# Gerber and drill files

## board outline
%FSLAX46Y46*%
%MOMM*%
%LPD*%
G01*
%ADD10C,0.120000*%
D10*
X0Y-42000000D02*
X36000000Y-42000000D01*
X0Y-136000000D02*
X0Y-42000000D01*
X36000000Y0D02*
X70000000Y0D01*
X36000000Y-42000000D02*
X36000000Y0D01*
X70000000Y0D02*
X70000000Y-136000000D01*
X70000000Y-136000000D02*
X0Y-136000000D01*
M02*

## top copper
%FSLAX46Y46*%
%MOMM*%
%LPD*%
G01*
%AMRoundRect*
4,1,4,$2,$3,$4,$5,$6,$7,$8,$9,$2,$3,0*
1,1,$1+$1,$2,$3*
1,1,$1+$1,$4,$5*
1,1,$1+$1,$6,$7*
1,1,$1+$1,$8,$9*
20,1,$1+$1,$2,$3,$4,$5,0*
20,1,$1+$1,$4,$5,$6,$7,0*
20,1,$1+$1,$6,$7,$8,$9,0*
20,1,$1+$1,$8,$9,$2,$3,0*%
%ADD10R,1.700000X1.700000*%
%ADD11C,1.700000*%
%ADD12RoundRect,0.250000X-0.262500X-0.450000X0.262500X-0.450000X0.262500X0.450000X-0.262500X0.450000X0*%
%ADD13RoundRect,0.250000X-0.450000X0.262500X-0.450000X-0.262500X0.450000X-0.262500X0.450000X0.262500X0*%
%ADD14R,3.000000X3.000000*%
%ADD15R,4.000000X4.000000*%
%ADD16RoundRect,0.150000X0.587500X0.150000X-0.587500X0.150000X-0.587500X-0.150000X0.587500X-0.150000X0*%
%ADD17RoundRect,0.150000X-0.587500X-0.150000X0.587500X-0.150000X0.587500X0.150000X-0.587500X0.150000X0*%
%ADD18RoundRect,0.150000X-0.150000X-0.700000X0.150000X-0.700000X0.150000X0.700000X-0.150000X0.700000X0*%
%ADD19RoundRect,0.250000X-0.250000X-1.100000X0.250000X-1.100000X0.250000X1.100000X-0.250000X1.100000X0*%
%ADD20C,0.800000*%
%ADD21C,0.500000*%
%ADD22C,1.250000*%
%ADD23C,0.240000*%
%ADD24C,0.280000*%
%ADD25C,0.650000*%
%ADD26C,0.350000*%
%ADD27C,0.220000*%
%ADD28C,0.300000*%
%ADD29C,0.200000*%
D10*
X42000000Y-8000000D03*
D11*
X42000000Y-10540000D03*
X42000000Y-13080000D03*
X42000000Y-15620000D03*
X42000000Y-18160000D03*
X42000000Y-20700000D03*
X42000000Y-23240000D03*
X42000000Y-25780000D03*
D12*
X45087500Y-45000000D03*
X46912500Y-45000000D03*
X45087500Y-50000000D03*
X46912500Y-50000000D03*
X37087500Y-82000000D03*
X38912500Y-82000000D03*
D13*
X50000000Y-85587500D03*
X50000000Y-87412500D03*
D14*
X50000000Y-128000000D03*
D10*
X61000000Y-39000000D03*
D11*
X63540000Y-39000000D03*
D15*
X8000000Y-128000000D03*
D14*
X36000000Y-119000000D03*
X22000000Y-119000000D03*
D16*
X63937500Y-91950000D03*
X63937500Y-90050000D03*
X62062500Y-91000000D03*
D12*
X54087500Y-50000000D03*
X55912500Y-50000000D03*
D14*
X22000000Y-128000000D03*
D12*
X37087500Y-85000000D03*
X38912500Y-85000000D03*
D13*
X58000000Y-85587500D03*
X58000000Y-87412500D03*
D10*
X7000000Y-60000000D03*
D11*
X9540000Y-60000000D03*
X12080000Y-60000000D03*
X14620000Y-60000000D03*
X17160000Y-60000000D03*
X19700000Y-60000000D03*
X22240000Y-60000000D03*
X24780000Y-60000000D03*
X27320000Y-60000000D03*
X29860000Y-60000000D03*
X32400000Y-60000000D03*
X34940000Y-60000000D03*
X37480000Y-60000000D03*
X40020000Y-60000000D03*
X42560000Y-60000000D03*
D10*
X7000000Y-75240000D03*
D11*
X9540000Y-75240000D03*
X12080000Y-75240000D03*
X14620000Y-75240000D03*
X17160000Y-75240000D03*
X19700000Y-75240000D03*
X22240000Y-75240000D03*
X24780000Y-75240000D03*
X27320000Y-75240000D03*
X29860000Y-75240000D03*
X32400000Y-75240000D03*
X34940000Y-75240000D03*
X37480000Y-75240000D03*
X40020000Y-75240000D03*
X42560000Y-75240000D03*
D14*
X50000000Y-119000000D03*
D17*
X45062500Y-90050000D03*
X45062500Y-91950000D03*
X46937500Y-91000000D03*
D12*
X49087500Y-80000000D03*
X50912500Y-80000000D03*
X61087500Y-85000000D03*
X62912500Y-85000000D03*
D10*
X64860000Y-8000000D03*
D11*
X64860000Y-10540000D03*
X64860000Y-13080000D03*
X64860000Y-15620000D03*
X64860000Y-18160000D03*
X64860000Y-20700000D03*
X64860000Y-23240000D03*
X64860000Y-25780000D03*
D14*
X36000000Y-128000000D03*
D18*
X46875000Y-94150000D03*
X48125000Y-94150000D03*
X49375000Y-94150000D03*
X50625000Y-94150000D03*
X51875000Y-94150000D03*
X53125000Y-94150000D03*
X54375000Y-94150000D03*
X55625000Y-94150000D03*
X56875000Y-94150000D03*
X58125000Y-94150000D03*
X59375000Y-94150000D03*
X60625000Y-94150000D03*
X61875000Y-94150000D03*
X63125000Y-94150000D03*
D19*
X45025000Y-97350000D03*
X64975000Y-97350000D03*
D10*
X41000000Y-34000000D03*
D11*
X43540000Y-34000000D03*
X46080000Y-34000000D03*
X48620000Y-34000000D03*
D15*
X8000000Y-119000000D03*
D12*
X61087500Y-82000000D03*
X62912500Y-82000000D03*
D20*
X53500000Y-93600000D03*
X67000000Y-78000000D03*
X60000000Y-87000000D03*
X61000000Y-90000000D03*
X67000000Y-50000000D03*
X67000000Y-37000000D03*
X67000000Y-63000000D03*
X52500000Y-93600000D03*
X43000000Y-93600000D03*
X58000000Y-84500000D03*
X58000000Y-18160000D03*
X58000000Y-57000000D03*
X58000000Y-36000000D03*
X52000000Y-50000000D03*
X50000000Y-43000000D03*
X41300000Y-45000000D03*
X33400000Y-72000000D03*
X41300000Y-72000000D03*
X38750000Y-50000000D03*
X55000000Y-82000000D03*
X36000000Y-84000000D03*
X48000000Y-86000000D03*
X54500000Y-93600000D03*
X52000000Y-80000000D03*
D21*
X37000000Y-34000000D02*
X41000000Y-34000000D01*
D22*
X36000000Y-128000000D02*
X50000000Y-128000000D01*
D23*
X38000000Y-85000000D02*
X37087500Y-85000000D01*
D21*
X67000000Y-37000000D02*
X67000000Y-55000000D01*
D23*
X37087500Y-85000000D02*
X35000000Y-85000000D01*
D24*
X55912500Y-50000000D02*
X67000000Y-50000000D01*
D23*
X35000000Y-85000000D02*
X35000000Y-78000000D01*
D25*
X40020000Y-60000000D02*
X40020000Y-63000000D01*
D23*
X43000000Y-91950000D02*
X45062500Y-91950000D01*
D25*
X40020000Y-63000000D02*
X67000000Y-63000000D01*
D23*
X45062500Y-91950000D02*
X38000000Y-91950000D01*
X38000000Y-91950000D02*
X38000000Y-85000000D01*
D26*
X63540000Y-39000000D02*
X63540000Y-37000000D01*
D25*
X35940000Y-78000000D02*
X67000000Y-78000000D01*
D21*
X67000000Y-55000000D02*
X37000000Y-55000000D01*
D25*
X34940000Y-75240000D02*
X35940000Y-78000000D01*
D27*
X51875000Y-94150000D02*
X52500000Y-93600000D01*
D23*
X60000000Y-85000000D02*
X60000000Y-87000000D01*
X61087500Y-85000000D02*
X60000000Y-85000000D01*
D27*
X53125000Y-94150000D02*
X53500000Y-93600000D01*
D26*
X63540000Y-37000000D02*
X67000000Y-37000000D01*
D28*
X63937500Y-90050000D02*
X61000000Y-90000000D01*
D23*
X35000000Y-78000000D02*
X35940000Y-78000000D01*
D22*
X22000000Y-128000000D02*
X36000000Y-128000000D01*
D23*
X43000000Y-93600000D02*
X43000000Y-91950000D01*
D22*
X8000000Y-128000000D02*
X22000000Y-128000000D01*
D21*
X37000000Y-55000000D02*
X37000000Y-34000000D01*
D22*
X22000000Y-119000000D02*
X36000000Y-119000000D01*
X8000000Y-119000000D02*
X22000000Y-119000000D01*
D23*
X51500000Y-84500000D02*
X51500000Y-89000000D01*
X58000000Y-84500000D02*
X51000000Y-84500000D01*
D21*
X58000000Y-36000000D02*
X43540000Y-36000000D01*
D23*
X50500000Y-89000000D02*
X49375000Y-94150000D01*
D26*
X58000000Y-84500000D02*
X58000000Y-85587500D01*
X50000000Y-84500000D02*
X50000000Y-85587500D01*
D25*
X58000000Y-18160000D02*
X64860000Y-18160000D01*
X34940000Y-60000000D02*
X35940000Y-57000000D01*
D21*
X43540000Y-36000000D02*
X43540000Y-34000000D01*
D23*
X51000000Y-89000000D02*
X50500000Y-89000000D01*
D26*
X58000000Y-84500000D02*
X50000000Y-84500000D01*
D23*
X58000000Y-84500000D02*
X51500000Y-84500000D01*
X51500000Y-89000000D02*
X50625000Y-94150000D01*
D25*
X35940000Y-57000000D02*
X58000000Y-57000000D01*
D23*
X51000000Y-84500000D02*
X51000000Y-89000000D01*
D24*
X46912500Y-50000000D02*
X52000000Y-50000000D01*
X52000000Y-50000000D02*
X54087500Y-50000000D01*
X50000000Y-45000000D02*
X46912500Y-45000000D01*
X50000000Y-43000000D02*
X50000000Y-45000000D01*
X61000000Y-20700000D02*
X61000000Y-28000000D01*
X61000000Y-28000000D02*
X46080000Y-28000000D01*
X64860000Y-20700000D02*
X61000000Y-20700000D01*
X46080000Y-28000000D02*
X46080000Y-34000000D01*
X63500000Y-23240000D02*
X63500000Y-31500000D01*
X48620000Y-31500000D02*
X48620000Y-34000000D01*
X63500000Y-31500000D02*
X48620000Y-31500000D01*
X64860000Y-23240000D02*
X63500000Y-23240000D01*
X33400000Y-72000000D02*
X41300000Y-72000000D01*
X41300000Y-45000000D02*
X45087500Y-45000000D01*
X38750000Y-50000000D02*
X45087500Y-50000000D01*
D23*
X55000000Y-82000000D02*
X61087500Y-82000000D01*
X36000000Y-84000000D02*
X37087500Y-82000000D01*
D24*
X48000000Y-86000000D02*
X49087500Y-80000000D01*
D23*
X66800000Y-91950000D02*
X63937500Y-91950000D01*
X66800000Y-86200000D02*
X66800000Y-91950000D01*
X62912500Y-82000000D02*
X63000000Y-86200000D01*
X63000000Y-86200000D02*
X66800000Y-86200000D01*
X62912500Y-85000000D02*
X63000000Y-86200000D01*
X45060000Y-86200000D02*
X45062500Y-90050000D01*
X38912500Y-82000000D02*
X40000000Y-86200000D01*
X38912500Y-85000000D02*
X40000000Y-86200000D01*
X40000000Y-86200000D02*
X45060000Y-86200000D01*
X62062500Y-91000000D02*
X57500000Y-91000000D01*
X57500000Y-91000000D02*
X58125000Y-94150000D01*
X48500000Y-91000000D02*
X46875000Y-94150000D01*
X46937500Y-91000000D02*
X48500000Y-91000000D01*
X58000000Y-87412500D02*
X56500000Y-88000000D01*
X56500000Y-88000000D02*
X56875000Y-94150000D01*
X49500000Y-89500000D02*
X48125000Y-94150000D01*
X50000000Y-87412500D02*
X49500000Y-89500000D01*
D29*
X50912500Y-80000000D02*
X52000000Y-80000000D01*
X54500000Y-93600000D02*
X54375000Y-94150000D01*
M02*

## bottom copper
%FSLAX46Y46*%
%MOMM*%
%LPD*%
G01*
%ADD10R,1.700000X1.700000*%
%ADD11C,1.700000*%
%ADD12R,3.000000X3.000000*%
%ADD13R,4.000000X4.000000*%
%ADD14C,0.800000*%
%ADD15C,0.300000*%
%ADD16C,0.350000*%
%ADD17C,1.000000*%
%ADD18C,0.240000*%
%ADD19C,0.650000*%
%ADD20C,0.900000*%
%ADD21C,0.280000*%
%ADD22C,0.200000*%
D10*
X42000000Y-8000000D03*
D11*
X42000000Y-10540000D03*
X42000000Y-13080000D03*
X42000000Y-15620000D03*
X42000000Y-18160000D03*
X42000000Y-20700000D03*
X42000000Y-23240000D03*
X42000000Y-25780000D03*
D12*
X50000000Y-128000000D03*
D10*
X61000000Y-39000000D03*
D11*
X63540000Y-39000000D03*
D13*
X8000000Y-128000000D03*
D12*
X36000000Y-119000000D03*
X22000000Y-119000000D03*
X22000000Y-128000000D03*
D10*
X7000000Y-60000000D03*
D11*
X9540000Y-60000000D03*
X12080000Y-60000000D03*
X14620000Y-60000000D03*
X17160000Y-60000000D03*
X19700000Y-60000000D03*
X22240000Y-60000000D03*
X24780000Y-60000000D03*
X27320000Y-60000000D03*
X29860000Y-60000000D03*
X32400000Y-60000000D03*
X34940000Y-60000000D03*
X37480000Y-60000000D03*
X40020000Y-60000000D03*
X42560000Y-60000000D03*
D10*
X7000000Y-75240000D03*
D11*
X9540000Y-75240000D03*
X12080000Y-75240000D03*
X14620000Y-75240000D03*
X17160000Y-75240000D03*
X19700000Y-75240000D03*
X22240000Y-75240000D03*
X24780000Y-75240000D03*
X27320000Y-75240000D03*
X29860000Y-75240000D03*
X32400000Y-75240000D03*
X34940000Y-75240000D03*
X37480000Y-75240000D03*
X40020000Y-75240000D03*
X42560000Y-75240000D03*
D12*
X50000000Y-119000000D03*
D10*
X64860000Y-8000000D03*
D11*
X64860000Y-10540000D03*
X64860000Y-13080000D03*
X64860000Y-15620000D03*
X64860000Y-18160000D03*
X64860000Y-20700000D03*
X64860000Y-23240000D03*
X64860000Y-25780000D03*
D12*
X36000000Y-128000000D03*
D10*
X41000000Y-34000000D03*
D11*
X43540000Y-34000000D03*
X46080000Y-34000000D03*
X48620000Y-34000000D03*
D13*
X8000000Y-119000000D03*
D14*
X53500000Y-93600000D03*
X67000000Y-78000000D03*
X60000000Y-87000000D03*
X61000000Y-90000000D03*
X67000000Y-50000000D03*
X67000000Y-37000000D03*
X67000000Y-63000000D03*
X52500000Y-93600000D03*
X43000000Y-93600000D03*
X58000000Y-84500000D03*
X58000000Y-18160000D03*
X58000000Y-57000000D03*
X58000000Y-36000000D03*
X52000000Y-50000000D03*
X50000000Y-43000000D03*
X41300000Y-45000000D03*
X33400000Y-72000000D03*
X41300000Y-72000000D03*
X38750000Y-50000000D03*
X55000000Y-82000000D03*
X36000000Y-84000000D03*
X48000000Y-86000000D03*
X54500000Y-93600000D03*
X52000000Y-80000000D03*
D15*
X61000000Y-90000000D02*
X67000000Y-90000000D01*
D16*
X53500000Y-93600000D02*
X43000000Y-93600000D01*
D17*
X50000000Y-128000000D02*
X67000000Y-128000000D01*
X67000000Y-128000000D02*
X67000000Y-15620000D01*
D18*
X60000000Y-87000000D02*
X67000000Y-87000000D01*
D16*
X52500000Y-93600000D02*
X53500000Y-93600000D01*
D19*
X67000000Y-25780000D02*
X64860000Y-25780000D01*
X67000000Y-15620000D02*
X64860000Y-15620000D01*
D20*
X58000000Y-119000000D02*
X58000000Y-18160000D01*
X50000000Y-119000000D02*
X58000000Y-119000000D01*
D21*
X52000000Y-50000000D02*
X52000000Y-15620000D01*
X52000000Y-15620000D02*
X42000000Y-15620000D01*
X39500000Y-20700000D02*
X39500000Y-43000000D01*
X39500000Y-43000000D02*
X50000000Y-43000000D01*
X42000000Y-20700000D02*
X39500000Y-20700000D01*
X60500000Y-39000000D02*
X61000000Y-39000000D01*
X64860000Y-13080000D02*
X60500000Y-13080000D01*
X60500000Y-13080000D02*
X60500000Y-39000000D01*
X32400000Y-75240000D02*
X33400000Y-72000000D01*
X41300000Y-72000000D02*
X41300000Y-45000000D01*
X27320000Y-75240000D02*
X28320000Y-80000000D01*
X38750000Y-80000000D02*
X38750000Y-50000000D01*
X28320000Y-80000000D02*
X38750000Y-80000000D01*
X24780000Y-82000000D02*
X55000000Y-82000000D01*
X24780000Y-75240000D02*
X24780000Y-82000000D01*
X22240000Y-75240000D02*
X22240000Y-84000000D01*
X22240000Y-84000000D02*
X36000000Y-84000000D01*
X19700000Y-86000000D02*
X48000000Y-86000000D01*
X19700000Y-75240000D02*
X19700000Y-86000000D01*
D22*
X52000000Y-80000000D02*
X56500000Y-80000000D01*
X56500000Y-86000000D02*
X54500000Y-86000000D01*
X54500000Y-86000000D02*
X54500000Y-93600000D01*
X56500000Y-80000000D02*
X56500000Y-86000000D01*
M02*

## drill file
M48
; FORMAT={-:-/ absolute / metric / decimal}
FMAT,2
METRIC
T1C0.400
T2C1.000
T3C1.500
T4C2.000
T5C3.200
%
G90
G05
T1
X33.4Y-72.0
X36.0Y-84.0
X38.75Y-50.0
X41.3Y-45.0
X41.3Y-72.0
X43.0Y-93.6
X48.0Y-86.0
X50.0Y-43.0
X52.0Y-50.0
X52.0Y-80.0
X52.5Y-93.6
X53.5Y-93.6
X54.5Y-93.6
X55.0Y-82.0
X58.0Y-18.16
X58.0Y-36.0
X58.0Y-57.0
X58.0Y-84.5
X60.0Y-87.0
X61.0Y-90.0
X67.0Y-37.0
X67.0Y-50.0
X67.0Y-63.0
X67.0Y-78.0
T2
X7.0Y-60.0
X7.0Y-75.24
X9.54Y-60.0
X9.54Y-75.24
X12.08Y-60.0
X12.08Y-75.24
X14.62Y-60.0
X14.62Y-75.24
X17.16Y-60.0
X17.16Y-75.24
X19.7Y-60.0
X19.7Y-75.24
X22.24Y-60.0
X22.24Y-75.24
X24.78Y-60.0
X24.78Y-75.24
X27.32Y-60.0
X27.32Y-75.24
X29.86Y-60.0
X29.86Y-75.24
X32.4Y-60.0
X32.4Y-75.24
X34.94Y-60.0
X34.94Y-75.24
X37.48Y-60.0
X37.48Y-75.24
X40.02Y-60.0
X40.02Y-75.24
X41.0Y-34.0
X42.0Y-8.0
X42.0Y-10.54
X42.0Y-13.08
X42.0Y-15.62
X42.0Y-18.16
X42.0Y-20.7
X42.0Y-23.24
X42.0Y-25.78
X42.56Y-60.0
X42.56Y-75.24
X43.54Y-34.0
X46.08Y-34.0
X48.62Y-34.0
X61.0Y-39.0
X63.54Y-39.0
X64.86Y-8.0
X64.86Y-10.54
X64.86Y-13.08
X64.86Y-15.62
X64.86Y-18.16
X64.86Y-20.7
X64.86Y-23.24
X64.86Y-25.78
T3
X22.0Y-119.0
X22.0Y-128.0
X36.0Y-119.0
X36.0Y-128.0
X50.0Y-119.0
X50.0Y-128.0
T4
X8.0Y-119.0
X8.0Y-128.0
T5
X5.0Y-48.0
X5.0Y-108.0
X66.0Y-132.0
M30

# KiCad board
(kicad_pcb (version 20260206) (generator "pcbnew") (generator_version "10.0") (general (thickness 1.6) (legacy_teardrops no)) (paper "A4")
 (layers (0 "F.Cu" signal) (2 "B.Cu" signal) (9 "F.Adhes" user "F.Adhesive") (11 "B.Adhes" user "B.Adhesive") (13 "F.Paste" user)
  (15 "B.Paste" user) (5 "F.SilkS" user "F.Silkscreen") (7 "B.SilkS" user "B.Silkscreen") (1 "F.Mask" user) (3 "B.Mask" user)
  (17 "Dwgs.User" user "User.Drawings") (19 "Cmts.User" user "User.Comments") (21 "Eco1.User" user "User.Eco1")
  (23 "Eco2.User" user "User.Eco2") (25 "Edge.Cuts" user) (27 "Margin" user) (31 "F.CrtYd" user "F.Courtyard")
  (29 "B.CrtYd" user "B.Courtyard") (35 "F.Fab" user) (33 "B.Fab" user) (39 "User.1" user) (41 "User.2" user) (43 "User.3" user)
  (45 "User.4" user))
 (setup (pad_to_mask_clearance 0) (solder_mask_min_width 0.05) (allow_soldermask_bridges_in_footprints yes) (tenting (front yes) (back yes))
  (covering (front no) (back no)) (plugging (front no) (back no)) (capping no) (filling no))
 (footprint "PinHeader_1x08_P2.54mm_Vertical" (layer "F.Cu") (at 42 8)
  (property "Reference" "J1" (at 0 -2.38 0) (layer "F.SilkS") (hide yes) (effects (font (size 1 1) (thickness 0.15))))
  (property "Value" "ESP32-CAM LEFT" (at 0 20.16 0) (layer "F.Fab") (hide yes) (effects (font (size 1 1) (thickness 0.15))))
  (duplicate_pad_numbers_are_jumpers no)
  (pad "1" thru_hole rect (at 0 0) (size 1.7 1.7) (drill 1) (layers "*.Cu" "*.Mask") (remove_unused_layers no))
  (pad "2" thru_hole circle (at 0 2.54) (size 1.7 1.7) (drill 1) (layers "*.Cu" "*.Mask") (remove_unused_layers no))
  (pad "3" thru_hole circle (at 0 5.08) (size 1.7 1.7) (drill 1) (layers "*.Cu" "*.Mask") (remove_unused_layers no))
  (pad "4" thru_hole circle (at 0 7.62) (size 1.7 1.7) (drill 1) (layers "*.Cu" "*.Mask") (remove_unused_layers no) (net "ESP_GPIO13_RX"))
  (pad "5" thru_hole circle (at 0 10.16) (size 1.7 1.7) (drill 1) (layers "*.Cu" "*.Mask") (remove_unused_layers no))
  (pad "6" thru_hole circle (at 0 12.7) (size 1.7 1.7) (drill 1) (layers "*.Cu" "*.Mask") (remove_unused_layers no) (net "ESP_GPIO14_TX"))
  (pad "7" thru_hole circle (at 0 15.24) (size 1.7 1.7) (drill 1) (layers "*.Cu" "*.Mask") (remove_unused_layers no))
  (pad "8" thru_hole circle (at 0 17.78) (size 1.7 1.7) (drill 1) (layers "*.Cu" "*.Mask") (remove_unused_layers no)))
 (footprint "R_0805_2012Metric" (layer "F.Cu") (at 46 45)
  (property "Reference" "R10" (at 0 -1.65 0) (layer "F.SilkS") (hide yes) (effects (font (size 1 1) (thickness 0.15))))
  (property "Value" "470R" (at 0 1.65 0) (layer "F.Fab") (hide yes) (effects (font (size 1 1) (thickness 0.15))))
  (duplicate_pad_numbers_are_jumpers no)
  (pad "1" smd roundrect (at -0.9125 0) (size 1.025 1.4) (layers "F.Cu" "F.Mask" "F.Paste") (roundrect_rratio 0.243902) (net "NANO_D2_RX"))
  (pad "2" smd roundrect (at 0.9125 0) (size 1.025 1.4) (layers "F.Cu" "F.Mask" "F.Paste") (roundrect_rratio 0.243902) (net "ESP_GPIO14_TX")))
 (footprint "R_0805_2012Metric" (layer "F.Cu") (at 46 50)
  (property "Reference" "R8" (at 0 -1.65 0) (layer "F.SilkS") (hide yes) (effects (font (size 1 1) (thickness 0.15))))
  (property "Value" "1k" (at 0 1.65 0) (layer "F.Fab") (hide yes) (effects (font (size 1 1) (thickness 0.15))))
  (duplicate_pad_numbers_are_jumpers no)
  (pad "1" smd roundrect (at -0.9125 0) (size 1.025 1.4) (layers "F.Cu" "F.Mask" "F.Paste") (roundrect_rratio 0.243902) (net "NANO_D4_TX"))
  (pad "2" smd roundrect (at 0.9125 0) (size 1.025 1.4) (layers "F.Cu" "F.Mask" "F.Paste") (roundrect_rratio 0.243902) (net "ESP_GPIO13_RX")))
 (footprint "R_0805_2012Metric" (layer "F.Cu") (at 38 82)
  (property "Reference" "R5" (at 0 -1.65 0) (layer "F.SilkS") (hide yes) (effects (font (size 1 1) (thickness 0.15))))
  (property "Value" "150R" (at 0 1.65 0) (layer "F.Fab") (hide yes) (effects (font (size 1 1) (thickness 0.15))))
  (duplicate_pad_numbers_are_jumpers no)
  (pad "1" smd roundrect (at -0.9125 0) (size 1.025 1.4) (layers "F.Cu" "F.Mask" "F.Paste") (roundrect_rratio 0.243902)
   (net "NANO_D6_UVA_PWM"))
  (pad "2" smd roundrect (at 0.9125 0) (size 1.025 1.4) (layers "F.Cu" "F.Mask" "F.Paste") (roundrect_rratio 0.243902) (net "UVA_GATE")))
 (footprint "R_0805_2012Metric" (layer "F.Cu") (at 50 86.5 -90)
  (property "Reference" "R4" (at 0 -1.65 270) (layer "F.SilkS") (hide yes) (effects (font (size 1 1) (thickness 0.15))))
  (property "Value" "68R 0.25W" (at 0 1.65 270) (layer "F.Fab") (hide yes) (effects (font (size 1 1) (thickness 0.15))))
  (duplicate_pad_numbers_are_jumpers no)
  (pad "1" smd roundrect (at -0.9125 0 270) (size 1.025 1.4) (layers "F.Cu" "F.Mask" "F.Paste") (roundrect_rratio 0.243902) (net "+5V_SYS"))
  (pad "2" smd roundrect (at 0.9125 0 270) (size 1.025 1.4) (layers "F.Cu" "F.Mask" "F.Paste") (roundrect_rratio 0.243902) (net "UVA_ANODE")))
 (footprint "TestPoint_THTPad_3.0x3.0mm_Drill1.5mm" (layer "F.Cu") (at 50 128)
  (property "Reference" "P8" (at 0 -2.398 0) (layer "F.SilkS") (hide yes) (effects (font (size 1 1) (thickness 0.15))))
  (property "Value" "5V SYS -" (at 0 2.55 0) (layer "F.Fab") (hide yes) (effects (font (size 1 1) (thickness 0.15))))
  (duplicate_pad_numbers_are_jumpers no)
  (pad "1" thru_hole rect (at 0 0) (size 3 3) (drill 1.5) (layers "*.Cu" "*.Mask") (remove_unused_layers no) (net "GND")))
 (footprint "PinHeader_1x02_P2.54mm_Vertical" (layer "F.Cu") (at 61 39 90)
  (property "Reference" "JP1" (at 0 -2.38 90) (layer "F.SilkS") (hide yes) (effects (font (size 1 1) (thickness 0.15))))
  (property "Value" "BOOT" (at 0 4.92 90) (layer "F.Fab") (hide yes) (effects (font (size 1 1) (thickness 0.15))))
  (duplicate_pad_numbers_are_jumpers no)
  (pad "1" thru_hole rect (at 0 0 90) (size 1.7 1.7) (drill 1) (layers "*.Cu" "*.Mask") (remove_unused_layers no) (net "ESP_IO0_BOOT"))
  (pad "2" thru_hole circle (at 0 2.54 90) (size 1.7 1.7) (drill 1) (layers "*.Cu" "*.Mask") (remove_unused_layers no) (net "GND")))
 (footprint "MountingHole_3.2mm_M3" (layer "F.Cu") (at 5 108)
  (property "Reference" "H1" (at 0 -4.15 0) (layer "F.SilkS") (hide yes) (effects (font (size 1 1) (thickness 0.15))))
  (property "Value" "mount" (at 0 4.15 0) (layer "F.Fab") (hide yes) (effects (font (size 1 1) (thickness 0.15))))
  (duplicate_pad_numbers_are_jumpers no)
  (pad "" np_thru_hole circle (at 0 0) (size 3.2 3.2) (drill 3.2) (layers "*.Cu" "*.Mask")))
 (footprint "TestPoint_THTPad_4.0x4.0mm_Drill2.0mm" (layer "F.Cu") (at 8 128)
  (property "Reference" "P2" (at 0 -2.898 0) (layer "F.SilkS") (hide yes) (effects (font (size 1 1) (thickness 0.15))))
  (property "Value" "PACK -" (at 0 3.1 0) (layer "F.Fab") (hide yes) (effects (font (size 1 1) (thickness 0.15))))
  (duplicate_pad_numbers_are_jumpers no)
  (pad "1" thru_hole rect (at 0 0) (size 4 4) (drill 2) (layers "*.Cu" "*.Mask") (remove_unused_layers no) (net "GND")))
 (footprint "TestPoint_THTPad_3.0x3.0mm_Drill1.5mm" (layer "F.Cu") (at 36 119)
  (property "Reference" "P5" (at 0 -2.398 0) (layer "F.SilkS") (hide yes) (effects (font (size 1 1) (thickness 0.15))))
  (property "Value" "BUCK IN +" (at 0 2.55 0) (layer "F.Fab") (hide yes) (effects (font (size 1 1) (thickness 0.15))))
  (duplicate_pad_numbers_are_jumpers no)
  (pad "1" thru_hole rect (at 0 0) (size 3 3) (drill 1.5) (layers "*.Cu" "*.Mask") (remove_unused_layers no) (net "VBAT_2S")))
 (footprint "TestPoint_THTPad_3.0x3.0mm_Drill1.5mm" (layer "F.Cu") (at 22 119)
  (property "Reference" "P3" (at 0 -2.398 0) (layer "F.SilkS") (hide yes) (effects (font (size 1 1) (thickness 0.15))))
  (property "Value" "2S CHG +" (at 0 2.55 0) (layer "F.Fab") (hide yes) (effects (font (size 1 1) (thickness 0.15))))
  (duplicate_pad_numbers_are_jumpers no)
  (pad "1" thru_hole rect (at 0 0) (size 3 3) (drill 1.5) (layers "*.Cu" "*.Mask") (remove_unused_layers no) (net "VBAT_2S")))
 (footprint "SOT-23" (layer "F.Cu") (at 63 91 180)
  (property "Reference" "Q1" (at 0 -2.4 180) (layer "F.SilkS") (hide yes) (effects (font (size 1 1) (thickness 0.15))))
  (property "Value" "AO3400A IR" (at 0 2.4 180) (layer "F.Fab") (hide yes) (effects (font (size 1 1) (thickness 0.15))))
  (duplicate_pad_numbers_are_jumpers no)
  (pad "1" smd roundrect (at -0.9375 -0.95 180) (size 1.475 0.6) (layers "F.Cu" "F.Mask" "F.Paste") (roundrect_rratio 0.25) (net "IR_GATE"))
  (pad "2" smd roundrect (at -0.9375 0.95 180) (size 1.475 0.6) (layers "F.Cu" "F.Mask" "F.Paste") (roundrect_rratio 0.25) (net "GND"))
  (pad "3" smd roundrect (at 0.9375 0 180) (size 1.475 0.6) (layers "F.Cu" "F.Mask" "F.Paste") (roundrect_rratio 0.25) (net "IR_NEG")))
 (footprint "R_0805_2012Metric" (layer "F.Cu") (at 55 50)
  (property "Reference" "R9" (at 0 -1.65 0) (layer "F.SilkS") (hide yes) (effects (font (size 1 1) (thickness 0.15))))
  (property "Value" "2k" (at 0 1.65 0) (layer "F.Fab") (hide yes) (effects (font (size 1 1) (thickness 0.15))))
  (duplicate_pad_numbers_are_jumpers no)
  (pad "1" smd roundrect (at -0.9125 0) (size 1.025 1.4) (layers "F.Cu" "F.Mask" "F.Paste") (roundrect_rratio 0.243902)
   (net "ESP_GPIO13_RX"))
  (pad "2" smd roundrect (at 0.9125 0) (size 1.025 1.4) (layers "F.Cu" "F.Mask" "F.Paste") (roundrect_rratio 0.243902) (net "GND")))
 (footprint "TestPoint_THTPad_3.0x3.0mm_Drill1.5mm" (layer "F.Cu") (at 22 128)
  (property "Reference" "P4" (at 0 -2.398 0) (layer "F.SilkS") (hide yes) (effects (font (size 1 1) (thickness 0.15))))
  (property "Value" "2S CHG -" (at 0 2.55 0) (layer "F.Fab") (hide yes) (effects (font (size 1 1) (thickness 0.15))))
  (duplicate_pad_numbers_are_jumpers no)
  (pad "1" thru_hole rect (at 0 0) (size 3 3) (drill 1.5) (layers "*.Cu" "*.Mask") (remove_unused_layers no) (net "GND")))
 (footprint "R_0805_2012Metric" (layer "F.Cu") (at 38 85)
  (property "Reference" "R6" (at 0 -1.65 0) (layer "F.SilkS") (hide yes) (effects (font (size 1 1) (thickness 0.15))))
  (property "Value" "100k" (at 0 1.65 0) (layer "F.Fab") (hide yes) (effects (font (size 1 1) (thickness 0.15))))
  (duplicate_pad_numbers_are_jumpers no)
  (pad "1" smd roundrect (at -0.9125 0) (size 1.025 1.4) (layers "F.Cu" "F.Mask" "F.Paste") (roundrect_rratio 0.243902) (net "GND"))
  (pad "2" smd roundrect (at 0.9125 0) (size 1.025 1.4) (layers "F.Cu" "F.Mask" "F.Paste") (roundrect_rratio 0.243902) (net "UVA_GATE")))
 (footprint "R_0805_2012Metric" (layer "F.Cu") (at 58 86.5 -90)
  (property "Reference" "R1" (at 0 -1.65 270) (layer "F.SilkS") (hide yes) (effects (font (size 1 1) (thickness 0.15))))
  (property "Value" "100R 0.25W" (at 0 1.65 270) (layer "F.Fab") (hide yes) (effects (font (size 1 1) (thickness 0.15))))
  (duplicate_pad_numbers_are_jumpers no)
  (pad "1" smd roundrect (at -0.9125 0 270) (size 1.025 1.4) (layers "F.Cu" "F.Mask" "F.Paste") (roundrect_rratio 0.243902) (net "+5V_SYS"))
  (pad "2" smd roundrect (at 0.9125 0 270) (size 1.025 1.4) (layers "F.Cu" "F.Mask" "F.Paste") (roundrect_rratio 0.243902) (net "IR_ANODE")))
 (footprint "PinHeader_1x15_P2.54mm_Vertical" (layer "F.Cu") (at 7 60 90)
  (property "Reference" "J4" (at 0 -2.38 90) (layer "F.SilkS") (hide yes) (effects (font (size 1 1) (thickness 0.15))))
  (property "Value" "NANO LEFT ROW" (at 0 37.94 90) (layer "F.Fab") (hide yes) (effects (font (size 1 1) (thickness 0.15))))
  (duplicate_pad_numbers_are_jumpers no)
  (pad "1" thru_hole rect (at 0 0 90) (size 1.7 1.7) (drill 1) (layers "*.Cu" "*.Mask") (remove_unused_layers no))
  (pad "2" thru_hole circle (at 0 2.54 90) (size 1.7 1.7) (drill 1) (layers "*.Cu" "*.Mask") (remove_unused_layers no))
  (pad "3" thru_hole circle (at 0 5.08 90) (size 1.7 1.7) (drill 1) (layers "*.Cu" "*.Mask") (remove_unused_layers no))
  (pad "4" thru_hole circle (at 0 7.62 90) (size 1.7 1.7) (drill 1) (layers "*.Cu" "*.Mask") (remove_unused_layers no))
  (pad "5" thru_hole circle (at 0 10.16 90) (size 1.7 1.7) (drill 1) (layers "*.Cu" "*.Mask") (remove_unused_layers no))
  (pad "6" thru_hole circle (at 0 12.7 90) (size 1.7 1.7) (drill 1) (layers "*.Cu" "*.Mask") (remove_unused_layers no))
  (pad "7" thru_hole circle (at 0 15.24 90) (size 1.7 1.7) (drill 1) (layers "*.Cu" "*.Mask") (remove_unused_layers no))
  (pad "8" thru_hole circle (at 0 17.78 90) (size 1.7 1.7) (drill 1) (layers "*.Cu" "*.Mask") (remove_unused_layers no))
  (pad "9" thru_hole circle (at 0 20.32 90) (size 1.7 1.7) (drill 1) (layers "*.Cu" "*.Mask") (remove_unused_layers no))
  (pad "10" thru_hole circle (at 0 22.86 90) (size 1.7 1.7) (drill 1) (layers "*.Cu" "*.Mask") (remove_unused_layers no))
  (pad "11" thru_hole circle (at 0 25.4 90) (size 1.7 1.7) (drill 1) (layers "*.Cu" "*.Mask") (remove_unused_layers no))
  (pad "12" thru_hole circle (at 0 27.94 90) (size 1.7 1.7) (drill 1) (layers "*.Cu" "*.Mask") (remove_unused_layers no) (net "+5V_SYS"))
  (pad "13" thru_hole circle (at 0 30.48 90) (size 1.7 1.7) (drill 1) (layers "*.Cu" "*.Mask") (remove_unused_layers no))
  (pad "14" thru_hole circle (at 0 33.02 90) (size 1.7 1.7) (drill 1) (layers "*.Cu" "*.Mask") (remove_unused_layers no) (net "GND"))
  (pad "15" thru_hole circle (at 0 35.56 90) (size 1.7 1.7) (drill 1) (layers "*.Cu" "*.Mask") (remove_unused_layers no)))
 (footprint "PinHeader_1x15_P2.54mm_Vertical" (layer "F.Cu") (at 7 75.24 90)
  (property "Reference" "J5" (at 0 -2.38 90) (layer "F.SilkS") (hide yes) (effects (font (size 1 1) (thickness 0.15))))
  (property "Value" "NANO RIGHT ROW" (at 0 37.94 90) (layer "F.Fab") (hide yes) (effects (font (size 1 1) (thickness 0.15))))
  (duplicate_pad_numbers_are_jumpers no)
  (pad "1" thru_hole rect (at 0 0 90) (size 1.7 1.7) (drill 1) (layers "*.Cu" "*.Mask") (remove_unused_layers no))
  (pad "2" thru_hole circle (at 0 2.54 90) (size 1.7 1.7) (drill 1) (layers "*.Cu" "*.Mask") (remove_unused_layers no))
  (pad "3" thru_hole circle (at 0 5.08 90) (size 1.7 1.7) (drill 1) (layers "*.Cu" "*.Mask") (remove_unused_layers no))
  (pad "4" thru_hole circle (at 0 7.62 90) (size 1.7 1.7) (drill 1) (layers "*.Cu" "*.Mask") (remove_unused_layers no))
  (pad "5" thru_hole circle (at 0 10.16 90) (size 1.7 1.7) (drill 1) (layers "*.Cu" "*.Mask") (remove_unused_layers no)
   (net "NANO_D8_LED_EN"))
  (pad "6" thru_hole circle (at 0 12.7 90) (size 1.7 1.7) (drill 1) (layers "*.Cu" "*.Mask") (remove_unused_layers no)
   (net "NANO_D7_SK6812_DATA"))
  (pad "7" thru_hole circle (at 0 15.24 90) (size 1.7 1.7) (drill 1) (layers "*.Cu" "*.Mask") (remove_unused_layers no)
   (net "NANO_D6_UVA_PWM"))
  (pad "8" thru_hole circle (at 0 17.78 90) (size 1.7 1.7) (drill 1) (layers "*.Cu" "*.Mask") (remove_unused_layers no)
   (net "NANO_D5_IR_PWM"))
  (pad "9" thru_hole circle (at 0 20.32 90) (size 1.7 1.7) (drill 1) (layers "*.Cu" "*.Mask") (remove_unused_layers no) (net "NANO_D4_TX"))
  (pad "10" thru_hole circle (at 0 22.86 90) (size 1.7 1.7) (drill 1) (layers "*.Cu" "*.Mask") (remove_unused_layers no))
  (pad "11" thru_hole circle (at 0 25.4 90) (size 1.7 1.7) (drill 1) (layers "*.Cu" "*.Mask") (remove_unused_layers no) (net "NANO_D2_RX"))
  (pad "12" thru_hole circle (at 0 27.94 90) (size 1.7 1.7) (drill 1) (layers "*.Cu" "*.Mask") (remove_unused_layers no) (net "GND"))
  (pad "13" thru_hole circle (at 0 30.48 90) (size 1.7 1.7) (drill 1) (layers "*.Cu" "*.Mask") (remove_unused_layers no))
  (pad "14" thru_hole circle (at 0 33.02 90) (size 1.7 1.7) (drill 1) (layers "*.Cu" "*.Mask") (remove_unused_layers no))
  (pad "15" thru_hole circle (at 0 35.56 90) (size 1.7 1.7) (drill 1) (layers "*.Cu" "*.Mask") (remove_unused_layers no)))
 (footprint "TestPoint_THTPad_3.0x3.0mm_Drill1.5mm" (layer "F.Cu") (at 50 119)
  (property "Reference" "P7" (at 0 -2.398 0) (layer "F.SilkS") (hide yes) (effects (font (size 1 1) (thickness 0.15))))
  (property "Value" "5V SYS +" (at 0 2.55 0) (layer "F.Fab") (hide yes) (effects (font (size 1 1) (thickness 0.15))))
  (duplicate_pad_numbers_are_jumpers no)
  (pad "1" thru_hole rect (at 0 0) (size 3 3) (drill 1.5) (layers "*.Cu" "*.Mask") (remove_unused_layers no) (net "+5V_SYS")))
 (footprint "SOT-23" (layer "F.Cu") (at 46 91)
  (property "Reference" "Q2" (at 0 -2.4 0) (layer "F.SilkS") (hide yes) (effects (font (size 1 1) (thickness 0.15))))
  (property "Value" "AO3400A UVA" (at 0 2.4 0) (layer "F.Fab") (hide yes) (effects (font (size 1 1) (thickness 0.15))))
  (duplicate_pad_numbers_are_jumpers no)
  (pad "1" smd roundrect (at -0.9375 -0.95) (size 1.475 0.6) (layers "F.Cu" "F.Mask" "F.Paste") (roundrect_rratio 0.25) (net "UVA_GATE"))
  (pad "2" smd roundrect (at -0.9375 0.95) (size 1.475 0.6) (layers "F.Cu" "F.Mask" "F.Paste") (roundrect_rratio 0.25) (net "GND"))
  (pad "3" smd roundrect (at 0.9375 0) (size 1.475 0.6) (layers "F.Cu" "F.Mask" "F.Paste") (roundrect_rratio 0.25) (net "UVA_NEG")))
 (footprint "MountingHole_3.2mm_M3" (layer "F.Cu") (at 66 132)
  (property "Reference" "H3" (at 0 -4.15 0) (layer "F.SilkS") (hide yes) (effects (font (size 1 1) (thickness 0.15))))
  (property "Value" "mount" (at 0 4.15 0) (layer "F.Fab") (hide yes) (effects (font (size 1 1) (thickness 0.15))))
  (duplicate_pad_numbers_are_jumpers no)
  (pad "" np_thru_hole circle (at 0 0) (size 3.2 3.2) (drill 3.2) (layers "*.Cu" "*.Mask")))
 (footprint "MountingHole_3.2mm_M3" (layer "F.Cu") (at 5 48)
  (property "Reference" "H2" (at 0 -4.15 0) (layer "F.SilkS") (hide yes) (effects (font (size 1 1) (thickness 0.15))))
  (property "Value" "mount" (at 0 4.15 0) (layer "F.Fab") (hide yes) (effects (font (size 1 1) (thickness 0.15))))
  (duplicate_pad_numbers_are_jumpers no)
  (pad "" np_thru_hole circle (at 0 0) (size 3.2 3.2) (drill 3.2) (layers "*.Cu" "*.Mask")))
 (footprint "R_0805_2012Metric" (layer "F.Cu") (at 50 80)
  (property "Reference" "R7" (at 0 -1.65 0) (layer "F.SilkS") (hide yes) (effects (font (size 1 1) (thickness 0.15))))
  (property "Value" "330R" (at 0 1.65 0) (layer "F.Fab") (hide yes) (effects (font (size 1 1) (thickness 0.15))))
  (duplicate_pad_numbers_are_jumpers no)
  (pad "1" smd roundrect (at -0.9125 0) (size 1.025 1.4) (layers "F.Cu" "F.Mask" "F.Paste") (roundrect_rratio 0.243902)
   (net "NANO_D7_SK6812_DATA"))
  (pad "2" smd roundrect (at 0.9125 0) (size 1.025 1.4) (layers "F.Cu" "F.Mask" "F.Paste") (roundrect_rratio 0.243902) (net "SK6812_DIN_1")))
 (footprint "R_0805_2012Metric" (layer "F.Cu") (at 62 85)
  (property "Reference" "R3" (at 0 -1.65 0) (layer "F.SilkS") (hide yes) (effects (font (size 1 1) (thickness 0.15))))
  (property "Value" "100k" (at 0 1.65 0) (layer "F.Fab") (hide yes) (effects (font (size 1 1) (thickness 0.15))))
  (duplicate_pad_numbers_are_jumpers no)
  (pad "1" smd roundrect (at -0.9125 0) (size 1.025 1.4) (layers "F.Cu" "F.Mask" "F.Paste") (roundrect_rratio 0.243902) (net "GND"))
  (pad "2" smd roundrect (at 0.9125 0) (size 1.025 1.4) (layers "F.Cu" "F.Mask" "F.Paste") (roundrect_rratio 0.243902) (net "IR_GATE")))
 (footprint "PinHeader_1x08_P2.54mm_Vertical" (layer "F.Cu") (at 64.86 8)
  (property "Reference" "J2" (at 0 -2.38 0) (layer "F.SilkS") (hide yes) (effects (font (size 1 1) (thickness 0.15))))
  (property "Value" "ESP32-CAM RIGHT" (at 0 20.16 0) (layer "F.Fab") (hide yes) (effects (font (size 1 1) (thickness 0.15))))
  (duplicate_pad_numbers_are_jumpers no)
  (pad "1" thru_hole rect (at 0 0) (size 1.7 1.7) (drill 1) (layers "*.Cu" "*.Mask") (remove_unused_layers no))
  (pad "2" thru_hole circle (at 0 2.54) (size 1.7 1.7) (drill 1) (layers "*.Cu" "*.Mask") (remove_unused_layers no))
  (pad "3" thru_hole circle (at 0 5.08) (size 1.7 1.7) (drill 1) (layers "*.Cu" "*.Mask") (remove_unused_layers no) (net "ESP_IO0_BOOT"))
  (pad "4" thru_hole circle (at 0 7.62) (size 1.7 1.7) (drill 1) (layers "*.Cu" "*.Mask") (remove_unused_layers no) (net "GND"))
  (pad "5" thru_hole circle (at 0 10.16) (size 1.7 1.7) (drill 1) (layers "*.Cu" "*.Mask") (remove_unused_layers no) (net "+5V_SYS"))
  (pad "6" thru_hole circle (at 0 12.7) (size 1.7 1.7) (drill 1) (layers "*.Cu" "*.Mask") (remove_unused_layers no) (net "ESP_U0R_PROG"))
  (pad "7" thru_hole circle (at 0 15.24) (size 1.7 1.7) (drill 1) (layers "*.Cu" "*.Mask") (remove_unused_layers no) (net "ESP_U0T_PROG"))
  (pad "8" thru_hole circle (at 0 17.78) (size 1.7 1.7) (drill 1) (layers "*.Cu" "*.Mask") (remove_unused_layers no) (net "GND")))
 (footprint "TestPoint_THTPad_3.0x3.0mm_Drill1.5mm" (layer "F.Cu") (at 36 128)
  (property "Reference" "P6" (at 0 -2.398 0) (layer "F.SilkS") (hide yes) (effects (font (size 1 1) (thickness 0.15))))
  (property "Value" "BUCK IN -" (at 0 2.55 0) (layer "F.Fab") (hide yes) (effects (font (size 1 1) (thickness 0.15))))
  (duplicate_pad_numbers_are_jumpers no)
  (pad "1" thru_hole rect (at 0 0) (size 3 3) (drill 1.5) (layers "*.Cu" "*.Mask") (remove_unused_layers no) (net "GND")))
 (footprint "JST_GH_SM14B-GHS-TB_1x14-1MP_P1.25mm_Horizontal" (layer "F.Cu") (at 55 96)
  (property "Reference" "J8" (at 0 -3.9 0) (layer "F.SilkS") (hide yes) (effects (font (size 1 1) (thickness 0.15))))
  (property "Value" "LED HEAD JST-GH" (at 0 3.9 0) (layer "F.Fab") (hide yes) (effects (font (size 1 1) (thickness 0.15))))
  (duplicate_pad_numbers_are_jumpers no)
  (pad "1" smd roundrect (at -8.125 -1.85) (size 0.6 1.7) (layers "F.Cu" "F.Mask" "F.Paste") (roundrect_rratio 0.25) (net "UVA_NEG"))
  (pad "2" smd roundrect (at -6.875 -1.85) (size 0.6 1.7) (layers "F.Cu" "F.Mask" "F.Paste") (roundrect_rratio 0.25) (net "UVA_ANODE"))
  (pad "3" smd roundrect (at -5.625 -1.85) (size 0.6 1.7) (layers "F.Cu" "F.Mask" "F.Paste") (roundrect_rratio 0.25) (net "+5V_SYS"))
  (pad "4" smd roundrect (at -4.375 -1.85) (size 0.6 1.7) (layers "F.Cu" "F.Mask" "F.Paste") (roundrect_rratio 0.25) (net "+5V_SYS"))
  (pad "5" smd roundrect (at -3.125 -1.85) (size 0.6 1.7) (layers "F.Cu" "F.Mask" "F.Paste") (roundrect_rratio 0.25) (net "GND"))
  (pad "6" smd roundrect (at -1.875 -1.85) (size 0.6 1.7) (layers "F.Cu" "F.Mask" "F.Paste") (roundrect_rratio 0.25) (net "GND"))
  (pad "7" smd roundrect (at -0.625 -1.85) (size 0.6 1.7) (layers "F.Cu" "F.Mask" "F.Paste") (roundrect_rratio 0.25) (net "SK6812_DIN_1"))
  (pad "8" smd roundrect (at 0.625 -1.85) (size 0.6 1.7) (layers "F.Cu" "F.Mask" "F.Paste") (roundrect_rratio 0.25))
  (pad "9" smd roundrect (at 1.875 -1.85) (size 0.6 1.7) (layers "F.Cu" "F.Mask" "F.Paste") (roundrect_rratio 0.25) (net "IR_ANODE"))
  (pad "10" smd roundrect (at 3.125 -1.85) (size 0.6 1.7) (layers "F.Cu" "F.Mask" "F.Paste") (roundrect_rratio 0.25) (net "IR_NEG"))
  (pad "11" smd roundrect (at 4.375 -1.85) (size 0.6 1.7) (layers "F.Cu" "F.Mask" "F.Paste") (roundrect_rratio 0.25))
  (pad "12" smd roundrect (at 5.625 -1.85) (size 0.6 1.7) (layers "F.Cu" "F.Mask" "F.Paste") (roundrect_rratio 0.25))
  (pad "13" smd roundrect (at 6.875 -1.85) (size 0.6 1.7) (layers "F.Cu" "F.Mask" "F.Paste") (roundrect_rratio 0.25))
  (pad "14" smd roundrect (at 8.125 -1.85) (size 0.6 1.7) (layers "F.Cu" "F.Mask" "F.Paste") (roundrect_rratio 0.25))
  (pad "MP" smd roundrect (at -9.975 1.35) (size 1 2.7) (layers "F.Cu" "F.Mask" "F.Paste") (roundrect_rratio 0.25))
  (pad "MP" smd roundrect (at 9.975 1.35) (size 1 2.7) (layers "F.Cu" "F.Mask" "F.Paste") (roundrect_rratio 0.25)))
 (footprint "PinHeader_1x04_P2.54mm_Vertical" (layer "F.Cu") (at 41 34 90)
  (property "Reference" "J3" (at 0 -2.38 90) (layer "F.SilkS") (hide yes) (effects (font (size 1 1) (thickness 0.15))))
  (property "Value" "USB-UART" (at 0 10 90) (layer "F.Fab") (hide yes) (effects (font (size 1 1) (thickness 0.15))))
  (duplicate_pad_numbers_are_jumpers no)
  (pad "1" thru_hole rect (at 0 0 90) (size 1.7 1.7) (drill 1) (layers "*.Cu" "*.Mask") (remove_unused_layers no) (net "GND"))
  (pad "2" thru_hole circle (at 0 2.54 90) (size 1.7 1.7) (drill 1) (layers "*.Cu" "*.Mask") (remove_unused_layers no) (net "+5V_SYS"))
  (pad "3" thru_hole circle (at 0 5.08 90) (size 1.7 1.7) (drill 1) (layers "*.Cu" "*.Mask") (remove_unused_layers no) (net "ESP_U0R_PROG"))
  (pad "4" thru_hole circle (at 0 7.62 90) (size 1.7 1.7) (drill 1) (layers "*.Cu" "*.Mask") (remove_unused_layers no) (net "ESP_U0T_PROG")))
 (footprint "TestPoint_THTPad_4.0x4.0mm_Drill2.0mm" (layer "F.Cu") (at 8 119)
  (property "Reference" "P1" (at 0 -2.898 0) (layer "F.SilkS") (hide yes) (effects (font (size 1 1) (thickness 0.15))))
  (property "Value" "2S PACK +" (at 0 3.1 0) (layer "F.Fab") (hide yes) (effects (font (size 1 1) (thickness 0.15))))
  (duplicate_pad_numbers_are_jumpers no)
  (pad "1" thru_hole rect (at 0 0) (size 4 4) (drill 2) (layers "*.Cu" "*.Mask") (remove_unused_layers no) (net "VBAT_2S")))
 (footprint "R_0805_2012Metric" (layer "F.Cu") (at 62 82)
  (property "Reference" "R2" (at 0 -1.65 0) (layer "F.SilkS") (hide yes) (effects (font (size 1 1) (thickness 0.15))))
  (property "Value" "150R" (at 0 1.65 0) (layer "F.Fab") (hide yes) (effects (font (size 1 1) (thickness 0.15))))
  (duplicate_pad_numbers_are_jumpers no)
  (pad "1" smd roundrect (at -0.9125 0) (size 1.025 1.4) (layers "F.Cu" "F.Mask" "F.Paste") (roundrect_rratio 0.243902)
   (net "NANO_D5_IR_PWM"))
  (pad "2" smd roundrect (at 0.9125 0) (size 1.025 1.4) (layers "F.Cu" "F.Mask" "F.Paste") (roundrect_rratio 0.243902) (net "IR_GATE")))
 (gr_line (start 0 42) (end 36 42) (stroke (width 0.12) (type default)) (layer "Edge.Cuts"))
 (gr_line (start 0 136) (end 0 42) (stroke (width 0.12) (type default)) (layer "Edge.Cuts"))
 (gr_line (start 36 0) (end 70 0) (stroke (width 0.12) (type default)) (layer "Edge.Cuts"))
 (gr_line (start 36 42) (end 36 0) (stroke (width 0.12) (type default)) (layer "Edge.Cuts"))
 (gr_line (start 70 0) (end 70 136) (stroke (width 0.12) (type default)) (layer "Edge.Cuts"))
 (gr_line (start 70 136) (end 0 136) (stroke (width 0.12) (type default)) (layer "Edge.Cuts"))
 (segment (start 37 34) (end 41 34) (width 0.5) (layer "F.Cu") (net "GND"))
 (segment (start 36 128) (end 50 128) (width 1.25) (layer "F.Cu") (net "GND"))
 (segment (start 38 85) (end 37.0875 85) (width 0.24) (layer "F.Cu") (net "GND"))
 (segment (start 67 37) (end 67 55) (width 0.5) (layer "F.Cu") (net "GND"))
 (segment (start 37.0875 85) (end 35 85) (width 0.24) (layer "F.Cu") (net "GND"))
 (segment (start 55.9125 50) (end 67 50) (width 0.28) (layer "F.Cu") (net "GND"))
 (segment (start 35 85) (end 35 78) (width 0.24) (layer "F.Cu") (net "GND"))
 (segment (start 40.02 60) (end 40.02 63) (width 0.65) (layer "F.Cu") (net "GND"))
 (segment (start 43 91.95) (end 45.0625 91.95) (width 0.24) (layer "F.Cu") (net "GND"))
 (segment (start 40.02 63) (end 67 63) (width 0.65) (layer "F.Cu") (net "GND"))
 (segment (start 45.0625 91.95) (end 38 91.95) (width 0.24) (layer "F.Cu") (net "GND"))
 (segment (start 38 91.95) (end 38 85) (width 0.24) (layer "F.Cu") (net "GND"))
 (segment (start 63.54 39) (end 63.54 37) (width 0.35) (layer "F.Cu") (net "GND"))
 (segment (start 35.94 78) (end 67 78) (width 0.65) (layer "F.Cu") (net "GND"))
 (segment (start 67 55) (end 37 55) (width 0.5) (layer "F.Cu") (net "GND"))
 (segment (start 34.94 75.24) (end 35.94 78) (width 0.65) (layer "F.Cu") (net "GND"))
 (segment (start 51.875 94.15) (end 52.5 93.6) (width 0.22) (layer "F.Cu") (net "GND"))
 (segment (start 60 85) (end 60 87) (width 0.24) (layer "F.Cu") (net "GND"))
 (segment (start 61.0875 85) (end 60 85) (width 0.24) (layer "F.Cu") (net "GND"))
 (segment (start 53.125 94.15) (end 53.5 93.6) (width 0.22) (layer "F.Cu") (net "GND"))
 (segment (start 63.54 37) (end 67 37) (width 0.35) (layer "F.Cu") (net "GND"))
 (segment (start 63.9375 90.05) (end 61 90) (width 0.3) (layer "F.Cu") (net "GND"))
 (segment (start 35 78) (end 35.94 78) (width 0.24) (layer "F.Cu") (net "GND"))
 (segment (start 22 128) (end 36 128) (width 1.25) (layer "F.Cu") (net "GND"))
 (segment (start 43 93.6) (end 43 91.95) (width 0.24) (layer "F.Cu") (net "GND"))
 (segment (start 8 128) (end 22 128) (width 1.25) (layer "F.Cu") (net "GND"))
 (segment (start 37 55) (end 37 34) (width 0.5) (layer "F.Cu") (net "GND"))
 (via (at 53.5 93.6) (size 0.8) (drill 0.4) (layers "F.Cu" "B.Cu") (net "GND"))
 (via (at 67 78) (size 0.8) (drill 0.4) (layers "F.Cu" "B.Cu") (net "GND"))
 (via (at 60 87) (size 0.8) (drill 0.4) (layers "F.Cu" "B.Cu") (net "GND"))
 (via (at 61 90) (size 0.8) (drill 0.4) (layers "F.Cu" "B.Cu") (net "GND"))
 (via (at 67 50) (size 0.8) (drill 0.4) (layers "F.Cu" "B.Cu") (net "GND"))
 (via (at 67 37) (size 0.8) (drill 0.4) (layers "F.Cu" "B.Cu") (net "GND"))
 (via (at 67 63) (size 0.8) (drill 0.4) (layers "F.Cu" "B.Cu") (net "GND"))
 (via (at 52.5 93.6) (size 0.8) (drill 0.4) (layers "F.Cu" "B.Cu") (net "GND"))
 (via (at 43 93.6) (size 0.8) (drill 0.4) (layers "F.Cu" "B.Cu") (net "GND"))
 (segment (start 61 90) (end 67 90) (width 0.3) (layer "B.Cu") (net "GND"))
 (segment (start 53.5 93.6) (end 43 93.6) (width 0.35) (layer "B.Cu") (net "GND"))
 (segment (start 50 128) (end 67 128) (width 1) (layer "B.Cu") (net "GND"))
 (segment (start 67 128) (end 67 15.62) (width 1) (layer "B.Cu") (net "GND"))
 (segment (start 60 87) (end 67 87) (width 0.24) (layer "B.Cu") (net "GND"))
 (segment (start 52.5 93.6) (end 53.5 93.6) (width 0.35) (layer "B.Cu") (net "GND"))
 (segment (start 67 25.78) (end 64.86 25.78) (width 0.65) (layer "B.Cu") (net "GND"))
 (segment (start 67 15.62) (end 64.86 15.62) (width 0.65) (layer "B.Cu") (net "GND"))
 (segment (start 22 119) (end 36 119) (width 1.25) (layer "F.Cu") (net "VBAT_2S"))
 (segment (start 8 119) (end 22 119) (width 1.25) (layer "F.Cu") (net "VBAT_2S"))
 (segment (start 51.5 84.5) (end 51.5 89) (width 0.24) (layer "F.Cu") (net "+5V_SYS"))
 (segment (start 58 84.5) (end 51 84.5) (width 0.24) (layer "F.Cu") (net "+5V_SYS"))
 (segment (start 58 36) (end 43.54 36) (width 0.5) (layer "F.Cu") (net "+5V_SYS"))
 (segment (start 50.5 89) (end 49.375 94.15) (width 0.24) (layer "F.Cu") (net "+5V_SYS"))
 (segment (start 58 84.5) (end 58 85.5875) (width 0.35) (layer "F.Cu") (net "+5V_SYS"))
 (segment (start 50 84.5) (end 50 85.5875) (width 0.35) (layer "F.Cu") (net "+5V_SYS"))
 (segment (start 58 18.16) (end 64.86 18.16) (width 0.65) (layer "F.Cu") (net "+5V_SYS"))
 (segment (start 34.94 60) (end 35.94 57) (width 0.65) (layer "F.Cu") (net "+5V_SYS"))
 (segment (start 43.54 36) (end 43.54 34) (width 0.5) (layer "F.Cu") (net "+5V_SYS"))
 (segment (start 51 89) (end 50.5 89) (width 0.24) (layer "F.Cu") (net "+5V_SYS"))
 (segment (start 58 84.5) (end 50 84.5) (width 0.35) (layer "F.Cu") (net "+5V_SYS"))
 (segment (start 58 84.5) (end 51.5 84.5) (width 0.24) (layer "F.Cu") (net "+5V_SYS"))
 (segment (start 51.5 89) (end 50.625 94.15) (width 0.24) (layer "F.Cu") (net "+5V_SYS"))
 (segment (start 35.94 57) (end 58 57) (width 0.65) (layer "F.Cu") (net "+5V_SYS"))
 (segment (start 51 84.5) (end 51 89) (width 0.24) (layer "F.Cu") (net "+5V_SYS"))
 (via (at 58 84.5) (size 0.8) (drill 0.4) (layers "F.Cu" "B.Cu") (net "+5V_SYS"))
 (via (at 58 18.16) (size 0.8) (drill 0.4) (layers "F.Cu" "B.Cu") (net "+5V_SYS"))
 (via (at 58 57) (size 0.8) (drill 0.4) (layers "F.Cu" "B.Cu") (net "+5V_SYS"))
 (via (at 58 36) (size 0.8) (drill 0.4) (layers "F.Cu" "B.Cu") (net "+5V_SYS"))
 (segment (start 58 119) (end 58 18.16) (width 0.9) (layer "B.Cu") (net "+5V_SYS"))
 (segment (start 50 119) (end 58 119) (width 0.9) (layer "B.Cu") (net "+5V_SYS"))
 (segment (start 46.9125 50) (end 52 50) (width 0.28) (layer "F.Cu") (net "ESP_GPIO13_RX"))
 (segment (start 52 50) (end 54.0875 50) (width 0.28) (layer "F.Cu") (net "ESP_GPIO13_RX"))
 (via (at 52 50) (size 0.8) (drill 0.4) (layers "F.Cu" "B.Cu") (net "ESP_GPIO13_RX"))
 (segment (start 52 50) (end 52 15.62) (width 0.28) (layer "B.Cu") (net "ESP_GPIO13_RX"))
 (segment (start 52 15.62) (end 42 15.62) (width 0.28) (layer "B.Cu") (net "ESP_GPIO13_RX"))
 (segment (start 50 45) (end 46.9125 45) (width 0.28) (layer "F.Cu") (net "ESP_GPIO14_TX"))
 (segment (start 50 43) (end 50 45) (width 0.28) (layer "F.Cu") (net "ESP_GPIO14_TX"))
 (via (at 50 43) (size 0.8) (drill 0.4) (layers "F.Cu" "B.Cu") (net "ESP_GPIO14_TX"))
 (segment (start 39.5 20.7) (end 39.5 43) (width 0.28) (layer "B.Cu") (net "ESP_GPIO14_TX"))
 (segment (start 39.5 43) (end 50 43) (width 0.28) (layer "B.Cu") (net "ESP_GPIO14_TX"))
 (segment (start 42 20.7) (end 39.5 20.7) (width 0.28) (layer "B.Cu") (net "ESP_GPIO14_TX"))
 (segment (start 61 20.7) (end 61 28) (width 0.28) (layer "F.Cu") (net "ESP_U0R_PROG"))
 (segment (start 61 28) (end 46.08 28) (width 0.28) (layer "F.Cu") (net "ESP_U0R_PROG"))
 (segment (start 64.86 20.7) (end 61 20.7) (width 0.28) (layer "F.Cu") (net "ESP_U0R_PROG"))
 (segment (start 46.08 28) (end 46.08 34) (width 0.28) (layer "F.Cu") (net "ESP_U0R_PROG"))
 (segment (start 63.5 23.24) (end 63.5 31.5) (width 0.28) (layer "F.Cu") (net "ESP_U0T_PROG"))
 (segment (start 48.62 31.5) (end 48.62 34) (width 0.28) (layer "F.Cu") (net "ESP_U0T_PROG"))
 (segment (start 63.5 31.5) (end 48.62 31.5) (width 0.28) (layer "F.Cu") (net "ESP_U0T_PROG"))
 (segment (start 64.86 23.24) (end 63.5 23.24) (width 0.28) (layer "F.Cu") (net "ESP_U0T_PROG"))
 (segment (start 60.5 39) (end 61 39) (width 0.28) (layer "B.Cu") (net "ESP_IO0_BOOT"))
 (segment (start 64.86 13.08) (end 60.5 13.08) (width 0.28) (layer "B.Cu") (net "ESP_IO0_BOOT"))
 (segment (start 60.5 13.08) (end 60.5 39) (width 0.28) (layer "B.Cu") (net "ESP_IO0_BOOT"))
 (segment (start 33.4 72) (end 41.3 72) (width 0.28) (layer "F.Cu") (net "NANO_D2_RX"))
 (segment (start 41.3 45) (end 45.0875 45) (width 0.28) (layer "F.Cu") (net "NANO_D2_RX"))
 (via (at 41.3 45) (size 0.8) (drill 0.4) (layers "F.Cu" "B.Cu") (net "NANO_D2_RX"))
 (via (at 33.4 72) (size 0.8) (drill 0.4) (layers "F.Cu" "B.Cu") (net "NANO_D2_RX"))
 (via (at 41.3 72) (size 0.8) (drill 0.4) (layers "F.Cu" "B.Cu") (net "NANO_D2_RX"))
 (segment (start 32.4 75.24) (end 33.4 72) (width 0.28) (layer "B.Cu") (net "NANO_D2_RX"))
 (segment (start 41.3 72) (end 41.3 45) (width 0.28) (layer "B.Cu") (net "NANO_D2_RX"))
 (segment (start 38.75 50) (end 45.0875 50) (width 0.28) (layer "F.Cu") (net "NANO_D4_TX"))
 (via (at 38.75 50) (size 0.8) (drill 0.4) (layers "F.Cu" "B.Cu") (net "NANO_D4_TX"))
 (segment (start 27.32 75.24) (end 28.32 80) (width 0.28) (layer "B.Cu") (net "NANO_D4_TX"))
 (segment (start 38.75 80) (end 38.75 50) (width 0.28) (layer "B.Cu") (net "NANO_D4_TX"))
 (segment (start 28.32 80) (end 38.75 80) (width 0.28) (layer "B.Cu") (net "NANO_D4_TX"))
 (segment (start 55 82) (end 61.0875 82) (width 0.24) (layer "F.Cu") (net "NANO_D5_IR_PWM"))
 (via (at 55 82) (size 0.8) (drill 0.4) (layers "F.Cu" "B.Cu") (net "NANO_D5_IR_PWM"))
 (segment (start 24.78 82) (end 55 82) (width 0.28) (layer "B.Cu") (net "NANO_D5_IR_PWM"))
 (segment (start 24.78 75.24) (end 24.78 82) (width 0.28) (layer "B.Cu") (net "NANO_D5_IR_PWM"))
 (segment (start 36 84) (end 37.0875 82) (width 0.24) (layer "F.Cu") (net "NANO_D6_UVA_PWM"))
 (via (at 36 84) (size 0.8) (drill 0.4) (layers "F.Cu" "B.Cu") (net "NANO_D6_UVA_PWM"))
 (segment (start 22.24 75.24) (end 22.24 84) (width 0.28) (layer "B.Cu") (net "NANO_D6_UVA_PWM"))
 (segment (start 22.24 84) (end 36 84) (width 0.28) (layer "B.Cu") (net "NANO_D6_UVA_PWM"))
 (segment (start 48 86) (end 49.0875 80) (width 0.28) (layer "F.Cu") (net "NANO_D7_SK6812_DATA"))
 (via (at 48 86) (size 0.8) (drill 0.4) (layers "F.Cu" "B.Cu") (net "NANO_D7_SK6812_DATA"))
 (segment (start 19.7 86) (end 48 86) (width 0.28) (layer "B.Cu") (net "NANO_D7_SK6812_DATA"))
 (segment (start 19.7 75.24) (end 19.7 86) (width 0.28) (layer "B.Cu") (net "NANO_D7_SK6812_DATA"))
 (segment (start 66.8 91.95) (end 63.9375 91.95) (width 0.24) (layer "F.Cu") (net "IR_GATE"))
 (segment (start 66.8 86.2) (end 66.8 91.95) (width 0.24) (layer "F.Cu") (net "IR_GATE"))
 (segment (start 62.9125 82) (end 63 86.2) (width 0.24) (layer "F.Cu") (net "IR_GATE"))
 (segment (start 63 86.2) (end 66.8 86.2) (width 0.24) (layer "F.Cu") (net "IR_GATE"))
 (segment (start 62.9125 85) (end 63 86.2) (width 0.24) (layer "F.Cu") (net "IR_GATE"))
 (segment (start 45.06 86.2) (end 45.0625 90.05) (width 0.24) (layer "F.Cu") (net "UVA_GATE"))
 (segment (start 38.9125 82) (end 40 86.2) (width 0.24) (layer "F.Cu") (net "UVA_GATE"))
 (segment (start 38.9125 85) (end 40 86.2) (width 0.24) (layer "F.Cu") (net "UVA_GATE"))
 (segment (start 40 86.2) (end 45.06 86.2) (width 0.24) (layer "F.Cu") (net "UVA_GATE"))
 (segment (start 62.0625 91) (end 57.5 91) (width 0.24) (layer "F.Cu") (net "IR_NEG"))
 (segment (start 57.5 91) (end 58.125 94.15) (width 0.24) (layer "F.Cu") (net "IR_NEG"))
 (segment (start 48.5 91) (end 46.875 94.15) (width 0.24) (layer "F.Cu") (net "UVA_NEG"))
 (segment (start 46.9375 91) (end 48.5 91) (width 0.24) (layer "F.Cu") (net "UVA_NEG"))
 (segment (start 58 87.4125) (end 56.5 88) (width 0.24) (layer "F.Cu") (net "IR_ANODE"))
 (segment (start 56.5 88) (end 56.875 94.15) (width 0.24) (layer "F.Cu") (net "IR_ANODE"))
 (segment (start 49.5 89.5) (end 48.125 94.15) (width 0.24) (layer "F.Cu") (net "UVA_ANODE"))
 (segment (start 50 87.4125) (end 49.5 89.5) (width 0.24) (layer "F.Cu") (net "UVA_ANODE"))
 (segment (start 50.9125 80) (end 52 80) (width 0.2) (layer "F.Cu") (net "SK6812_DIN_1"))
 (segment (start 54.5 93.6) (end 54.375 94.15) (width 0.2) (layer "F.Cu") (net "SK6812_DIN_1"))
 (via (at 54.5 93.6) (size 0.8) (drill 0.4) (layers "F.Cu" "B.Cu") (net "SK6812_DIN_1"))
 (via (at 52 80) (size 0.8) (drill 0.4) (layers "F.Cu" "B.Cu") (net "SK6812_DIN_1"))
 (segment (start 52 80) (end 56.5 80) (width 0.2) (layer "B.Cu") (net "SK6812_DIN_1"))
 (segment (start 56.5 86) (end 54.5 86) (width 0.2) (layer "B.Cu") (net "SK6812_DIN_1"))
 (segment (start 54.5 86) (end 54.5 93.6) (width 0.2) (layer "B.Cu") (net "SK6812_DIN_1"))
 (segment (start 56.5 80) (end 56.5 86) (width 0.2) (layer "B.Cu") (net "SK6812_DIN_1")))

